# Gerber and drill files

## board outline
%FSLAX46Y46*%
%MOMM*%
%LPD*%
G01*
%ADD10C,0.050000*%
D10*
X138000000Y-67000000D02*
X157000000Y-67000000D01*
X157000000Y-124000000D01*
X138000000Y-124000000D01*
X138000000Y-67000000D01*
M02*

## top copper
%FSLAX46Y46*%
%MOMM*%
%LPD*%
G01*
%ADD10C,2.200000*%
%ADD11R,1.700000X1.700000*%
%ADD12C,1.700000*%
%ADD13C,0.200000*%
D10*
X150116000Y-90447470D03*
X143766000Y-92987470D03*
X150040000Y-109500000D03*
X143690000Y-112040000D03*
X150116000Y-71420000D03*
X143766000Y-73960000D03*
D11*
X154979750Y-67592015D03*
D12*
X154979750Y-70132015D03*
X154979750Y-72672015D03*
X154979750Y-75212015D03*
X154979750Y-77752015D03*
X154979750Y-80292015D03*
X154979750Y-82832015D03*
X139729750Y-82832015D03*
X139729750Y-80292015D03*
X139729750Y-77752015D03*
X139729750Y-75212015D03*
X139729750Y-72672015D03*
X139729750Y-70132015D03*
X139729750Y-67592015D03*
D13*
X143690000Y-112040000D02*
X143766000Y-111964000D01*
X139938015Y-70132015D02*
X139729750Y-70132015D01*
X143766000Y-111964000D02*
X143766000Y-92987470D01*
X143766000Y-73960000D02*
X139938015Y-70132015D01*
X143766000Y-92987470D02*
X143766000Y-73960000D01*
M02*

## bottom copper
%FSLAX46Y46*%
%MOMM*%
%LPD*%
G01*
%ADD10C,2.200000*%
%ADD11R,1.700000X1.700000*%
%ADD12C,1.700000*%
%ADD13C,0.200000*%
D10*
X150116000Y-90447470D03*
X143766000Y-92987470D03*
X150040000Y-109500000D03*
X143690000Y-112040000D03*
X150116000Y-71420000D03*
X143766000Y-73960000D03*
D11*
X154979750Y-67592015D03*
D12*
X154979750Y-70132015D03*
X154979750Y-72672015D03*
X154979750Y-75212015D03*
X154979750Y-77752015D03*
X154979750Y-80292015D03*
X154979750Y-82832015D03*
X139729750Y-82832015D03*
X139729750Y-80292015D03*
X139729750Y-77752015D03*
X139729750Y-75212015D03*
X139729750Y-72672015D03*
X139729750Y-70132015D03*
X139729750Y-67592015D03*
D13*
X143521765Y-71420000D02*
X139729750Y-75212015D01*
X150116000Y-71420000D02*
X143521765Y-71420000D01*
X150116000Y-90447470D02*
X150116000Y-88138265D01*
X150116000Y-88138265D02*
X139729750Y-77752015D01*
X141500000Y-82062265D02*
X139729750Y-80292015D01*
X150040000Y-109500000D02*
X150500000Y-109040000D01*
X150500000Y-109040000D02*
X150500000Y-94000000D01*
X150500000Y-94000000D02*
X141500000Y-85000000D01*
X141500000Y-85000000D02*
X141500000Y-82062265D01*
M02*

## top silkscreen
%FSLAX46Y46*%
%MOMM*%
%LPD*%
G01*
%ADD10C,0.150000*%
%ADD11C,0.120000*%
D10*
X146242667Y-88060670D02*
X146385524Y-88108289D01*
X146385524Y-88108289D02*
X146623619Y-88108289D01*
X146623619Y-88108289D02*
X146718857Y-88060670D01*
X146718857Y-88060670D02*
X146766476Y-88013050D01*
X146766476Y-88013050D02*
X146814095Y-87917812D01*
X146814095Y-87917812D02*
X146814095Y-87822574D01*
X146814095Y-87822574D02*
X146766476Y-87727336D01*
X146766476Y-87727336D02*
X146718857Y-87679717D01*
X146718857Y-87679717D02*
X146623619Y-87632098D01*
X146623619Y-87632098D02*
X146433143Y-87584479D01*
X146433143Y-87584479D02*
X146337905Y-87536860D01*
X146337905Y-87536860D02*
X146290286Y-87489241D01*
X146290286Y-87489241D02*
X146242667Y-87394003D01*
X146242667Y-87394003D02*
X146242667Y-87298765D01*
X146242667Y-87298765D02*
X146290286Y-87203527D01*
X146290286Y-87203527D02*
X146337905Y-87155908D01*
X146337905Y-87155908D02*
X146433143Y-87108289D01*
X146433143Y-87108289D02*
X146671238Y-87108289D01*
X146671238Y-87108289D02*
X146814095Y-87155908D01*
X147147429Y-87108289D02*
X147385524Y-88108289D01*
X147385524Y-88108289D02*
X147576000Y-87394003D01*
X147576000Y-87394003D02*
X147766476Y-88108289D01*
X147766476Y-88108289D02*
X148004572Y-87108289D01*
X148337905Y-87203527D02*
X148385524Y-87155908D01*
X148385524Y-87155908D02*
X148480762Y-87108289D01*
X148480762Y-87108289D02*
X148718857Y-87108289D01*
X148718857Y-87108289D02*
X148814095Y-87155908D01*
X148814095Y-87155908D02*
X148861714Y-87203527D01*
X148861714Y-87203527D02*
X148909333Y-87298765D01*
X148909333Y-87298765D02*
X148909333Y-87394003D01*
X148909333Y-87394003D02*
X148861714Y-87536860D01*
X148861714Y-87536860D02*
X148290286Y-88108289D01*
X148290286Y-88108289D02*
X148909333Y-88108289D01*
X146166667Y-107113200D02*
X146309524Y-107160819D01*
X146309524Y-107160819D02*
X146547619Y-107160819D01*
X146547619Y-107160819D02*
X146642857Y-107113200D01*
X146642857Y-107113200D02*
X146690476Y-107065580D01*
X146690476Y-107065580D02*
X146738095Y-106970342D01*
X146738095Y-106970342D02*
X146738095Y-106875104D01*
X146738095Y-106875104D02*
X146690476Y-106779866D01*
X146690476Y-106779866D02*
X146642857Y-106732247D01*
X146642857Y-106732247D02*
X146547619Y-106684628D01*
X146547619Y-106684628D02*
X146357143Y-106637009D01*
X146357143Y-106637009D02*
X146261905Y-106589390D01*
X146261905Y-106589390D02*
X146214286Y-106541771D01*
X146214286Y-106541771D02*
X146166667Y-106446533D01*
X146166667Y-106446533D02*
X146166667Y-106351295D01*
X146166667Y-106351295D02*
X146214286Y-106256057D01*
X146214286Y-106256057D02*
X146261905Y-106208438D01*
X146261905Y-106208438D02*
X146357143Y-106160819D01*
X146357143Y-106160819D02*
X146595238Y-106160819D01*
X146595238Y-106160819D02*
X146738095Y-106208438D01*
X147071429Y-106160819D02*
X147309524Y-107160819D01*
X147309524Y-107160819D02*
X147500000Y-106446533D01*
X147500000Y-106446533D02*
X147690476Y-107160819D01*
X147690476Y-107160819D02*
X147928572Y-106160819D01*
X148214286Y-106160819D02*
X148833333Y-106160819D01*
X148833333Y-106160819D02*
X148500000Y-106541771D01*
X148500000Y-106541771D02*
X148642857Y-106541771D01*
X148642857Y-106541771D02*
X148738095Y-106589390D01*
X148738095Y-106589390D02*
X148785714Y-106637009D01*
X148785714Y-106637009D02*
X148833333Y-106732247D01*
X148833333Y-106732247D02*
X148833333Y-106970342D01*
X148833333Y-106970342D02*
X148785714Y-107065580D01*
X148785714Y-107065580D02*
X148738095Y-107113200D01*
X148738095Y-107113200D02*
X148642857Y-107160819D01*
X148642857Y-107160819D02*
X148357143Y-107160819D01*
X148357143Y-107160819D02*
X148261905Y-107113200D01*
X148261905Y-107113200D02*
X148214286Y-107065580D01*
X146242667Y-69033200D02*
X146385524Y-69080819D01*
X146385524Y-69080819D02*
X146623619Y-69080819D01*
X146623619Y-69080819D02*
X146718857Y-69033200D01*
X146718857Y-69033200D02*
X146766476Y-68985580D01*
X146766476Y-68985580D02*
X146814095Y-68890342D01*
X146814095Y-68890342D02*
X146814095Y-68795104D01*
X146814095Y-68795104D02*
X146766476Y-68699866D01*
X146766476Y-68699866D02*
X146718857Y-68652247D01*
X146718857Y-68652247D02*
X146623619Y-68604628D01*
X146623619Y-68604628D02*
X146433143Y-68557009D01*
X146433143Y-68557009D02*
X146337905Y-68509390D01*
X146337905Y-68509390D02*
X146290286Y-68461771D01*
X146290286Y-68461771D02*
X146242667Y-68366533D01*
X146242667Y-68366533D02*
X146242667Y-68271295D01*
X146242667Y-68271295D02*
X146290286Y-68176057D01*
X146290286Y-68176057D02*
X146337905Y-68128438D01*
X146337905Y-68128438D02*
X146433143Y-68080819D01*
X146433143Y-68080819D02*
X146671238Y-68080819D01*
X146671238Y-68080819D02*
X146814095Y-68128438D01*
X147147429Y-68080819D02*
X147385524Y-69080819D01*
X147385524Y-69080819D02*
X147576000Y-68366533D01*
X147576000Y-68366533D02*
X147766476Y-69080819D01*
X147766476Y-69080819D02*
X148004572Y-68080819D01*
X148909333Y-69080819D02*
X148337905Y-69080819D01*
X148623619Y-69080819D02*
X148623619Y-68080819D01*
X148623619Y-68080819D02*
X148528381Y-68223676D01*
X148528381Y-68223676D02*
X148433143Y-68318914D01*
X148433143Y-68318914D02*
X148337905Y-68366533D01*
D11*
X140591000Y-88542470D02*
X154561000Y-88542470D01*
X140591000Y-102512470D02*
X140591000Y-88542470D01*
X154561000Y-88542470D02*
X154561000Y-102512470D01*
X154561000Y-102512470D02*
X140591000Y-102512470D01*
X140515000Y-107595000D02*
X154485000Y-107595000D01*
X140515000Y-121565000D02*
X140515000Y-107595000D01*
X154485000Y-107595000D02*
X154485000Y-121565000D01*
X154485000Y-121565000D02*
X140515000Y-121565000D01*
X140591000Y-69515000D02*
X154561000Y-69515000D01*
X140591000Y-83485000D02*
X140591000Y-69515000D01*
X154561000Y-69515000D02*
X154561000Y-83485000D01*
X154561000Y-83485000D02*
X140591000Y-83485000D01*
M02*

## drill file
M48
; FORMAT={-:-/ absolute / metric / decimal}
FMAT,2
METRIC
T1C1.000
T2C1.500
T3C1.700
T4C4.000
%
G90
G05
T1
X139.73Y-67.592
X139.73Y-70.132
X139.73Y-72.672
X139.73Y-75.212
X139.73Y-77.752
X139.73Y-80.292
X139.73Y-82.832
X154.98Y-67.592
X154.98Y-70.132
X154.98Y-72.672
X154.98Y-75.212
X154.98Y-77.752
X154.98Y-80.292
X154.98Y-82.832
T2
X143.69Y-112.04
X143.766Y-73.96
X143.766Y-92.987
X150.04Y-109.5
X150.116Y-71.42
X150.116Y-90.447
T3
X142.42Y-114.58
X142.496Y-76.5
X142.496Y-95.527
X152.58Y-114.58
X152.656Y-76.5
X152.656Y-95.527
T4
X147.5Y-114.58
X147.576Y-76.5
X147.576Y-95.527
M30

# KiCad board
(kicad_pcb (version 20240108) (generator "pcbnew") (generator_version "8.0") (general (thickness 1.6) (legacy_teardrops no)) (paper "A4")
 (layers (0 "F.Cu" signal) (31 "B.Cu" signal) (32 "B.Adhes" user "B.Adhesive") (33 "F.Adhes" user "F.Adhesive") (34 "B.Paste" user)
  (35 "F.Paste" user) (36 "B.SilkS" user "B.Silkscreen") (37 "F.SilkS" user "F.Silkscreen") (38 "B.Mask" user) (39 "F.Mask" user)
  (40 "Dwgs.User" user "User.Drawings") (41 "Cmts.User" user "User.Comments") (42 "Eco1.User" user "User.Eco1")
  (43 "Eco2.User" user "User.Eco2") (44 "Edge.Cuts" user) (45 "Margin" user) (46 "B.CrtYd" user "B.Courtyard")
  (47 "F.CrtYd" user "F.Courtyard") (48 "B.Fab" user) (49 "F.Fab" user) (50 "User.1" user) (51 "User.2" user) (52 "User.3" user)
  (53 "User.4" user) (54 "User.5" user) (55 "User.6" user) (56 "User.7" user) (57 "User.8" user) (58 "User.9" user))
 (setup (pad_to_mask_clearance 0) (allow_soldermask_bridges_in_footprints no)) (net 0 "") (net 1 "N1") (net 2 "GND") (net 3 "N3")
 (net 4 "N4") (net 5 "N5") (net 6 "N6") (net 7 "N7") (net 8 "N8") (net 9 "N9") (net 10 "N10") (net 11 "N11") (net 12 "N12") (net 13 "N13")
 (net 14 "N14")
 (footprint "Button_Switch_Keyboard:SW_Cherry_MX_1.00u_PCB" (layer "F.Cu") (at 150.116 90.44747)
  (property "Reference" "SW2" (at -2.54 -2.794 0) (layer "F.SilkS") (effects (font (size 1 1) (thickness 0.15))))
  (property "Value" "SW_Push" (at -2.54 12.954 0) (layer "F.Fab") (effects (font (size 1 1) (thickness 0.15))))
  (fp_line (start -9.525 -1.905) (end 4.445 -1.905) (stroke (width 0.12) (type solid)) (layer "F.SilkS"))
  (fp_line (start -9.525 12.065) (end -9.525 -1.905) (stroke (width 0.12) (type solid)) (layer "F.SilkS"))
  (fp_line (start 4.445 -1.905) (end 4.445 12.065) (stroke (width 0.12) (type solid)) (layer "F.SilkS"))
  (fp_line (start 4.445 12.065) (end -9.525 12.065) (stroke (width 0.12) (type solid)) (layer "F.SilkS"))
  (pad "" np_thru_hole circle (at -7.62 5.08) (size 1.7 1.7) (drill 1.7) (layers "*.Cu" "*.Mask"))
  (pad "" np_thru_hole circle (at -2.54 5.08) (size 4 4) (drill 4) (layers "*.Cu" "*.Mask"))
  (pad "" np_thru_hole circle (at 2.54 5.08) (size 1.7 1.7) (drill 1.7) (layers "*.Cu" "*.Mask"))
  (pad "1" thru_hole circle (at 0 0) (size 2.2 2.2) (drill 1.5) (layers "*.Cu" "*.Mask") (remove_unused_layers no) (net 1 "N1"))
  (pad "2" thru_hole circle (at -6.35 2.54) (size 2.2 2.2) (drill 1.5) (layers "*.Cu" "*.Mask") (remove_unused_layers no) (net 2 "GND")))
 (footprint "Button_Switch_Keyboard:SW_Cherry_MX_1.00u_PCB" (layer "F.Cu") (at 150.04 109.5)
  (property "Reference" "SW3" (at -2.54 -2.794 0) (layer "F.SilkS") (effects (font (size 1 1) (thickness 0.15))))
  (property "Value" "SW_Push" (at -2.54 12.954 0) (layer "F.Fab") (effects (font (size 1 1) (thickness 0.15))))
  (fp_line (start -9.525 -1.905) (end 4.445 -1.905) (stroke (width 0.12) (type solid)) (layer "F.SilkS"))
  (fp_line (start -9.525 12.065) (end -9.525 -1.905) (stroke (width 0.12) (type solid)) (layer "F.SilkS"))
  (fp_line (start 4.445 -1.905) (end 4.445 12.065) (stroke (width 0.12) (type solid)) (layer "F.SilkS"))
  (fp_line (start 4.445 12.065) (end -9.525 12.065) (stroke (width 0.12) (type solid)) (layer "F.SilkS"))
  (pad "" np_thru_hole circle (at -7.62 5.08) (size 1.7 1.7) (drill 1.7) (layers "*.Cu" "*.Mask"))
  (pad "" np_thru_hole circle (at -2.54 5.08) (size 4 4) (drill 4) (layers "*.Cu" "*.Mask"))
  (pad "" np_thru_hole circle (at 2.54 5.08) (size 1.7 1.7) (drill 1.7) (layers "*.Cu" "*.Mask"))
  (pad "1" thru_hole circle (at 0 0) (size 2.2 2.2) (drill 1.5) (layers "*.Cu" "*.Mask") (remove_unused_layers no) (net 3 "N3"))
  (pad "2" thru_hole circle (at -6.35 2.54) (size 2.2 2.2) (drill 1.5) (layers "*.Cu" "*.Mask") (remove_unused_layers no) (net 2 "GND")))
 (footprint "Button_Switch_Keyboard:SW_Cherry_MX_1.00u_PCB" (layer "F.Cu") (at 150.116 71.42)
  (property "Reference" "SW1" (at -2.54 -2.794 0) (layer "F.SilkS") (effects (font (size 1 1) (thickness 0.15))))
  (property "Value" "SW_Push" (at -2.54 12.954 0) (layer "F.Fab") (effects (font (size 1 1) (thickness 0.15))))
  (fp_line (start -9.525 -1.905) (end 4.445 -1.905) (stroke (width 0.12) (type solid)) (layer "F.SilkS"))
  (fp_line (start -9.525 12.065) (end -9.525 -1.905) (stroke (width 0.12) (type solid)) (layer "F.SilkS"))
  (fp_line (start 4.445 -1.905) (end 4.445 12.065) (stroke (width 0.12) (type solid)) (layer "F.SilkS"))
  (fp_line (start 4.445 12.065) (end -9.525 12.065) (stroke (width 0.12) (type solid)) (layer "F.SilkS"))
  (pad "" np_thru_hole circle (at -7.62 5.08) (size 1.7 1.7) (drill 1.7) (layers "*.Cu" "*.Mask"))
  (pad "" np_thru_hole circle (at -2.54 5.08) (size 4 4) (drill 4) (layers "*.Cu" "*.Mask"))
  (pad "" np_thru_hole circle (at 2.54 5.08) (size 1.7 1.7) (drill 1.7) (layers "*.Cu" "*.Mask"))
  (pad "1" thru_hole circle (at 0 0) (size 2.2 2.2) (drill 1.5) (layers "*.Cu" "*.Mask") (remove_unused_layers no) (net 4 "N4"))
  (pad "2" thru_hole circle (at -6.35 2.54) (size 2.2 2.2) (drill 1.5) (layers "*.Cu" "*.Mask") (remove_unused_layers no) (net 2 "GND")))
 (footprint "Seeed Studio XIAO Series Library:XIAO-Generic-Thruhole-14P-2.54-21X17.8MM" (layer "B.Cu") (at 147.35475 75.212015 180)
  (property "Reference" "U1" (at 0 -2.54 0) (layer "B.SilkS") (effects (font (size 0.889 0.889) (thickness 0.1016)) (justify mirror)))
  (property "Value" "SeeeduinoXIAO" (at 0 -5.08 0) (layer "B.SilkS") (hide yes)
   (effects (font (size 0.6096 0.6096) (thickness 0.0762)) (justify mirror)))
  (pad "1" thru_hole rect (at -7.625 7.62 180) (size 1.7 1.7) (drill 1) (layers "*.Cu" "*.Mask") (remove_unused_layers no) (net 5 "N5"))
  (pad "2" thru_hole circle (at -7.625 5.08 180) (size 1.7 1.7) (drill 1) (layers "*.Cu" "*.Mask") (remove_unused_layers no) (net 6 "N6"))
  (pad "3" thru_hole circle (at -7.625 2.54 180) (size 1.7 1.7) (drill 1) (layers "*.Cu" "*.Mask") (remove_unused_layers no) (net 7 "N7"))
  (pad "4" thru_hole circle (at -7.625 0 180) (size 1.7 1.7) (drill 1) (layers "*.Cu" "*.Mask") (remove_unused_layers no) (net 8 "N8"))
  (pad "5" thru_hole circle (at -7.625 -2.54 180) (size 1.7 1.7) (drill 1) (layers "*.Cu" "*.Mask") (remove_unused_layers no) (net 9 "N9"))
  (pad "6" thru_hole circle (at -7.625 -5.08) (size 1.7 1.7) (drill 1) (layers "*.Cu" "*.Mask") (remove_unused_layers no) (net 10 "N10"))
  (pad "7" thru_hole circle (at -7.625 -7.62 180) (size 1.7 1.7) (drill 1) (layers "*.Cu" "*.Mask") (remove_unused_layers no) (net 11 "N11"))
  (pad "8" thru_hole circle (at 7.625 -7.62 180) (size 1.7 1.7) (drill 1) (layers "*.Cu" "*.Mask") (remove_unused_layers no) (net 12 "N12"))
  (pad "9" thru_hole circle (at 7.625 -5.08 180) (size 1.7 1.7) (drill 1) (layers "*.Cu" "*.Mask") (remove_unused_layers no) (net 3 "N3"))
  (pad "10" thru_hole circle (at 7.625 -2.54 180) (size 1.7 1.7) (drill 1) (layers "*.Cu" "*.Mask") (remove_unused_layers no) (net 1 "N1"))
  (pad "11" thru_hole circle (at 7.625 0 180) (size 1.7 1.7) (drill 1) (layers "*.Cu" "*.Mask") (remove_unused_layers no) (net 4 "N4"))
  (pad "12" thru_hole circle (at 7.625 2.54 180) (size 1.7 1.7) (drill 1) (layers "*.Cu" "*.Mask") (remove_unused_layers no) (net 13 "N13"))
  (pad "13" thru_hole circle (at 7.625 5.08 180) (size 1.7 1.7) (drill 1) (layers "*.Cu" "*.Mask") (remove_unused_layers no) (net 2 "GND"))
  (pad "14" thru_hole circle (at 7.625 7.62 180) (size 1.7 1.7) (drill 1) (layers "*.Cu" "*.Mask") (remove_unused_layers no) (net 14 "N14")))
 (gr_rect (start 138 67) (end 157 124) (stroke (width 0.05) (type default)) (fill none) (layer "Edge.Cuts"))
 (segment (start 143.69 112.04) (end 143.766 111.964) (width 0.2) (layer "F.Cu") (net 2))
 (segment (start 139.938015 70.132015) (end 139.72975 70.132015) (width 0.2) (layer "F.Cu") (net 2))
 (segment (start 143.766 111.964) (end 143.766 92.98747) (width 0.2) (layer "F.Cu") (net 2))
 (segment (start 143.766 73.96) (end 139.938015 70.132015) (width 0.2) (layer "F.Cu") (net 2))
 (segment (start 143.766 92.98747) (end 143.766 73.96) (width 0.2) (layer "F.Cu") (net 2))
 (segment (start 143.521765 71.42) (end 139.72975 75.212015) (width 0.2) (layer "B.Cu") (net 4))
 (segment (start 150.116 71.42) (end 143.521765 71.42) (width 0.2) (layer "B.Cu") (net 4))
 (segment (start 150.116 90.44747) (end 150.116 88.138265) (width 0.2) (layer "B.Cu") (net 1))
 (segment (start 150.116 88.138265) (end 139.72975 77.752015) (width 0.2) (layer "B.Cu") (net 1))
 (segment (start 141.5 82.062265) (end 139.72975 80.292015) (width 0.2) (layer "B.Cu") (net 3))
 (segment (start 150.04 109.5) (end 150.5 109.04) (width 0.2) (layer "B.Cu") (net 3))
 (segment (start 150.5 109.04) (end 150.5 94) (width 0.2) (layer "B.Cu") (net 3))
 (segment (start 150.5 94) (end 141.5 85) (width 0.2) (layer "B.Cu") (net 3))
 (segment (start 141.5 85) (end 141.5 82.062265) (width 0.2) (layer "B.Cu") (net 3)))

